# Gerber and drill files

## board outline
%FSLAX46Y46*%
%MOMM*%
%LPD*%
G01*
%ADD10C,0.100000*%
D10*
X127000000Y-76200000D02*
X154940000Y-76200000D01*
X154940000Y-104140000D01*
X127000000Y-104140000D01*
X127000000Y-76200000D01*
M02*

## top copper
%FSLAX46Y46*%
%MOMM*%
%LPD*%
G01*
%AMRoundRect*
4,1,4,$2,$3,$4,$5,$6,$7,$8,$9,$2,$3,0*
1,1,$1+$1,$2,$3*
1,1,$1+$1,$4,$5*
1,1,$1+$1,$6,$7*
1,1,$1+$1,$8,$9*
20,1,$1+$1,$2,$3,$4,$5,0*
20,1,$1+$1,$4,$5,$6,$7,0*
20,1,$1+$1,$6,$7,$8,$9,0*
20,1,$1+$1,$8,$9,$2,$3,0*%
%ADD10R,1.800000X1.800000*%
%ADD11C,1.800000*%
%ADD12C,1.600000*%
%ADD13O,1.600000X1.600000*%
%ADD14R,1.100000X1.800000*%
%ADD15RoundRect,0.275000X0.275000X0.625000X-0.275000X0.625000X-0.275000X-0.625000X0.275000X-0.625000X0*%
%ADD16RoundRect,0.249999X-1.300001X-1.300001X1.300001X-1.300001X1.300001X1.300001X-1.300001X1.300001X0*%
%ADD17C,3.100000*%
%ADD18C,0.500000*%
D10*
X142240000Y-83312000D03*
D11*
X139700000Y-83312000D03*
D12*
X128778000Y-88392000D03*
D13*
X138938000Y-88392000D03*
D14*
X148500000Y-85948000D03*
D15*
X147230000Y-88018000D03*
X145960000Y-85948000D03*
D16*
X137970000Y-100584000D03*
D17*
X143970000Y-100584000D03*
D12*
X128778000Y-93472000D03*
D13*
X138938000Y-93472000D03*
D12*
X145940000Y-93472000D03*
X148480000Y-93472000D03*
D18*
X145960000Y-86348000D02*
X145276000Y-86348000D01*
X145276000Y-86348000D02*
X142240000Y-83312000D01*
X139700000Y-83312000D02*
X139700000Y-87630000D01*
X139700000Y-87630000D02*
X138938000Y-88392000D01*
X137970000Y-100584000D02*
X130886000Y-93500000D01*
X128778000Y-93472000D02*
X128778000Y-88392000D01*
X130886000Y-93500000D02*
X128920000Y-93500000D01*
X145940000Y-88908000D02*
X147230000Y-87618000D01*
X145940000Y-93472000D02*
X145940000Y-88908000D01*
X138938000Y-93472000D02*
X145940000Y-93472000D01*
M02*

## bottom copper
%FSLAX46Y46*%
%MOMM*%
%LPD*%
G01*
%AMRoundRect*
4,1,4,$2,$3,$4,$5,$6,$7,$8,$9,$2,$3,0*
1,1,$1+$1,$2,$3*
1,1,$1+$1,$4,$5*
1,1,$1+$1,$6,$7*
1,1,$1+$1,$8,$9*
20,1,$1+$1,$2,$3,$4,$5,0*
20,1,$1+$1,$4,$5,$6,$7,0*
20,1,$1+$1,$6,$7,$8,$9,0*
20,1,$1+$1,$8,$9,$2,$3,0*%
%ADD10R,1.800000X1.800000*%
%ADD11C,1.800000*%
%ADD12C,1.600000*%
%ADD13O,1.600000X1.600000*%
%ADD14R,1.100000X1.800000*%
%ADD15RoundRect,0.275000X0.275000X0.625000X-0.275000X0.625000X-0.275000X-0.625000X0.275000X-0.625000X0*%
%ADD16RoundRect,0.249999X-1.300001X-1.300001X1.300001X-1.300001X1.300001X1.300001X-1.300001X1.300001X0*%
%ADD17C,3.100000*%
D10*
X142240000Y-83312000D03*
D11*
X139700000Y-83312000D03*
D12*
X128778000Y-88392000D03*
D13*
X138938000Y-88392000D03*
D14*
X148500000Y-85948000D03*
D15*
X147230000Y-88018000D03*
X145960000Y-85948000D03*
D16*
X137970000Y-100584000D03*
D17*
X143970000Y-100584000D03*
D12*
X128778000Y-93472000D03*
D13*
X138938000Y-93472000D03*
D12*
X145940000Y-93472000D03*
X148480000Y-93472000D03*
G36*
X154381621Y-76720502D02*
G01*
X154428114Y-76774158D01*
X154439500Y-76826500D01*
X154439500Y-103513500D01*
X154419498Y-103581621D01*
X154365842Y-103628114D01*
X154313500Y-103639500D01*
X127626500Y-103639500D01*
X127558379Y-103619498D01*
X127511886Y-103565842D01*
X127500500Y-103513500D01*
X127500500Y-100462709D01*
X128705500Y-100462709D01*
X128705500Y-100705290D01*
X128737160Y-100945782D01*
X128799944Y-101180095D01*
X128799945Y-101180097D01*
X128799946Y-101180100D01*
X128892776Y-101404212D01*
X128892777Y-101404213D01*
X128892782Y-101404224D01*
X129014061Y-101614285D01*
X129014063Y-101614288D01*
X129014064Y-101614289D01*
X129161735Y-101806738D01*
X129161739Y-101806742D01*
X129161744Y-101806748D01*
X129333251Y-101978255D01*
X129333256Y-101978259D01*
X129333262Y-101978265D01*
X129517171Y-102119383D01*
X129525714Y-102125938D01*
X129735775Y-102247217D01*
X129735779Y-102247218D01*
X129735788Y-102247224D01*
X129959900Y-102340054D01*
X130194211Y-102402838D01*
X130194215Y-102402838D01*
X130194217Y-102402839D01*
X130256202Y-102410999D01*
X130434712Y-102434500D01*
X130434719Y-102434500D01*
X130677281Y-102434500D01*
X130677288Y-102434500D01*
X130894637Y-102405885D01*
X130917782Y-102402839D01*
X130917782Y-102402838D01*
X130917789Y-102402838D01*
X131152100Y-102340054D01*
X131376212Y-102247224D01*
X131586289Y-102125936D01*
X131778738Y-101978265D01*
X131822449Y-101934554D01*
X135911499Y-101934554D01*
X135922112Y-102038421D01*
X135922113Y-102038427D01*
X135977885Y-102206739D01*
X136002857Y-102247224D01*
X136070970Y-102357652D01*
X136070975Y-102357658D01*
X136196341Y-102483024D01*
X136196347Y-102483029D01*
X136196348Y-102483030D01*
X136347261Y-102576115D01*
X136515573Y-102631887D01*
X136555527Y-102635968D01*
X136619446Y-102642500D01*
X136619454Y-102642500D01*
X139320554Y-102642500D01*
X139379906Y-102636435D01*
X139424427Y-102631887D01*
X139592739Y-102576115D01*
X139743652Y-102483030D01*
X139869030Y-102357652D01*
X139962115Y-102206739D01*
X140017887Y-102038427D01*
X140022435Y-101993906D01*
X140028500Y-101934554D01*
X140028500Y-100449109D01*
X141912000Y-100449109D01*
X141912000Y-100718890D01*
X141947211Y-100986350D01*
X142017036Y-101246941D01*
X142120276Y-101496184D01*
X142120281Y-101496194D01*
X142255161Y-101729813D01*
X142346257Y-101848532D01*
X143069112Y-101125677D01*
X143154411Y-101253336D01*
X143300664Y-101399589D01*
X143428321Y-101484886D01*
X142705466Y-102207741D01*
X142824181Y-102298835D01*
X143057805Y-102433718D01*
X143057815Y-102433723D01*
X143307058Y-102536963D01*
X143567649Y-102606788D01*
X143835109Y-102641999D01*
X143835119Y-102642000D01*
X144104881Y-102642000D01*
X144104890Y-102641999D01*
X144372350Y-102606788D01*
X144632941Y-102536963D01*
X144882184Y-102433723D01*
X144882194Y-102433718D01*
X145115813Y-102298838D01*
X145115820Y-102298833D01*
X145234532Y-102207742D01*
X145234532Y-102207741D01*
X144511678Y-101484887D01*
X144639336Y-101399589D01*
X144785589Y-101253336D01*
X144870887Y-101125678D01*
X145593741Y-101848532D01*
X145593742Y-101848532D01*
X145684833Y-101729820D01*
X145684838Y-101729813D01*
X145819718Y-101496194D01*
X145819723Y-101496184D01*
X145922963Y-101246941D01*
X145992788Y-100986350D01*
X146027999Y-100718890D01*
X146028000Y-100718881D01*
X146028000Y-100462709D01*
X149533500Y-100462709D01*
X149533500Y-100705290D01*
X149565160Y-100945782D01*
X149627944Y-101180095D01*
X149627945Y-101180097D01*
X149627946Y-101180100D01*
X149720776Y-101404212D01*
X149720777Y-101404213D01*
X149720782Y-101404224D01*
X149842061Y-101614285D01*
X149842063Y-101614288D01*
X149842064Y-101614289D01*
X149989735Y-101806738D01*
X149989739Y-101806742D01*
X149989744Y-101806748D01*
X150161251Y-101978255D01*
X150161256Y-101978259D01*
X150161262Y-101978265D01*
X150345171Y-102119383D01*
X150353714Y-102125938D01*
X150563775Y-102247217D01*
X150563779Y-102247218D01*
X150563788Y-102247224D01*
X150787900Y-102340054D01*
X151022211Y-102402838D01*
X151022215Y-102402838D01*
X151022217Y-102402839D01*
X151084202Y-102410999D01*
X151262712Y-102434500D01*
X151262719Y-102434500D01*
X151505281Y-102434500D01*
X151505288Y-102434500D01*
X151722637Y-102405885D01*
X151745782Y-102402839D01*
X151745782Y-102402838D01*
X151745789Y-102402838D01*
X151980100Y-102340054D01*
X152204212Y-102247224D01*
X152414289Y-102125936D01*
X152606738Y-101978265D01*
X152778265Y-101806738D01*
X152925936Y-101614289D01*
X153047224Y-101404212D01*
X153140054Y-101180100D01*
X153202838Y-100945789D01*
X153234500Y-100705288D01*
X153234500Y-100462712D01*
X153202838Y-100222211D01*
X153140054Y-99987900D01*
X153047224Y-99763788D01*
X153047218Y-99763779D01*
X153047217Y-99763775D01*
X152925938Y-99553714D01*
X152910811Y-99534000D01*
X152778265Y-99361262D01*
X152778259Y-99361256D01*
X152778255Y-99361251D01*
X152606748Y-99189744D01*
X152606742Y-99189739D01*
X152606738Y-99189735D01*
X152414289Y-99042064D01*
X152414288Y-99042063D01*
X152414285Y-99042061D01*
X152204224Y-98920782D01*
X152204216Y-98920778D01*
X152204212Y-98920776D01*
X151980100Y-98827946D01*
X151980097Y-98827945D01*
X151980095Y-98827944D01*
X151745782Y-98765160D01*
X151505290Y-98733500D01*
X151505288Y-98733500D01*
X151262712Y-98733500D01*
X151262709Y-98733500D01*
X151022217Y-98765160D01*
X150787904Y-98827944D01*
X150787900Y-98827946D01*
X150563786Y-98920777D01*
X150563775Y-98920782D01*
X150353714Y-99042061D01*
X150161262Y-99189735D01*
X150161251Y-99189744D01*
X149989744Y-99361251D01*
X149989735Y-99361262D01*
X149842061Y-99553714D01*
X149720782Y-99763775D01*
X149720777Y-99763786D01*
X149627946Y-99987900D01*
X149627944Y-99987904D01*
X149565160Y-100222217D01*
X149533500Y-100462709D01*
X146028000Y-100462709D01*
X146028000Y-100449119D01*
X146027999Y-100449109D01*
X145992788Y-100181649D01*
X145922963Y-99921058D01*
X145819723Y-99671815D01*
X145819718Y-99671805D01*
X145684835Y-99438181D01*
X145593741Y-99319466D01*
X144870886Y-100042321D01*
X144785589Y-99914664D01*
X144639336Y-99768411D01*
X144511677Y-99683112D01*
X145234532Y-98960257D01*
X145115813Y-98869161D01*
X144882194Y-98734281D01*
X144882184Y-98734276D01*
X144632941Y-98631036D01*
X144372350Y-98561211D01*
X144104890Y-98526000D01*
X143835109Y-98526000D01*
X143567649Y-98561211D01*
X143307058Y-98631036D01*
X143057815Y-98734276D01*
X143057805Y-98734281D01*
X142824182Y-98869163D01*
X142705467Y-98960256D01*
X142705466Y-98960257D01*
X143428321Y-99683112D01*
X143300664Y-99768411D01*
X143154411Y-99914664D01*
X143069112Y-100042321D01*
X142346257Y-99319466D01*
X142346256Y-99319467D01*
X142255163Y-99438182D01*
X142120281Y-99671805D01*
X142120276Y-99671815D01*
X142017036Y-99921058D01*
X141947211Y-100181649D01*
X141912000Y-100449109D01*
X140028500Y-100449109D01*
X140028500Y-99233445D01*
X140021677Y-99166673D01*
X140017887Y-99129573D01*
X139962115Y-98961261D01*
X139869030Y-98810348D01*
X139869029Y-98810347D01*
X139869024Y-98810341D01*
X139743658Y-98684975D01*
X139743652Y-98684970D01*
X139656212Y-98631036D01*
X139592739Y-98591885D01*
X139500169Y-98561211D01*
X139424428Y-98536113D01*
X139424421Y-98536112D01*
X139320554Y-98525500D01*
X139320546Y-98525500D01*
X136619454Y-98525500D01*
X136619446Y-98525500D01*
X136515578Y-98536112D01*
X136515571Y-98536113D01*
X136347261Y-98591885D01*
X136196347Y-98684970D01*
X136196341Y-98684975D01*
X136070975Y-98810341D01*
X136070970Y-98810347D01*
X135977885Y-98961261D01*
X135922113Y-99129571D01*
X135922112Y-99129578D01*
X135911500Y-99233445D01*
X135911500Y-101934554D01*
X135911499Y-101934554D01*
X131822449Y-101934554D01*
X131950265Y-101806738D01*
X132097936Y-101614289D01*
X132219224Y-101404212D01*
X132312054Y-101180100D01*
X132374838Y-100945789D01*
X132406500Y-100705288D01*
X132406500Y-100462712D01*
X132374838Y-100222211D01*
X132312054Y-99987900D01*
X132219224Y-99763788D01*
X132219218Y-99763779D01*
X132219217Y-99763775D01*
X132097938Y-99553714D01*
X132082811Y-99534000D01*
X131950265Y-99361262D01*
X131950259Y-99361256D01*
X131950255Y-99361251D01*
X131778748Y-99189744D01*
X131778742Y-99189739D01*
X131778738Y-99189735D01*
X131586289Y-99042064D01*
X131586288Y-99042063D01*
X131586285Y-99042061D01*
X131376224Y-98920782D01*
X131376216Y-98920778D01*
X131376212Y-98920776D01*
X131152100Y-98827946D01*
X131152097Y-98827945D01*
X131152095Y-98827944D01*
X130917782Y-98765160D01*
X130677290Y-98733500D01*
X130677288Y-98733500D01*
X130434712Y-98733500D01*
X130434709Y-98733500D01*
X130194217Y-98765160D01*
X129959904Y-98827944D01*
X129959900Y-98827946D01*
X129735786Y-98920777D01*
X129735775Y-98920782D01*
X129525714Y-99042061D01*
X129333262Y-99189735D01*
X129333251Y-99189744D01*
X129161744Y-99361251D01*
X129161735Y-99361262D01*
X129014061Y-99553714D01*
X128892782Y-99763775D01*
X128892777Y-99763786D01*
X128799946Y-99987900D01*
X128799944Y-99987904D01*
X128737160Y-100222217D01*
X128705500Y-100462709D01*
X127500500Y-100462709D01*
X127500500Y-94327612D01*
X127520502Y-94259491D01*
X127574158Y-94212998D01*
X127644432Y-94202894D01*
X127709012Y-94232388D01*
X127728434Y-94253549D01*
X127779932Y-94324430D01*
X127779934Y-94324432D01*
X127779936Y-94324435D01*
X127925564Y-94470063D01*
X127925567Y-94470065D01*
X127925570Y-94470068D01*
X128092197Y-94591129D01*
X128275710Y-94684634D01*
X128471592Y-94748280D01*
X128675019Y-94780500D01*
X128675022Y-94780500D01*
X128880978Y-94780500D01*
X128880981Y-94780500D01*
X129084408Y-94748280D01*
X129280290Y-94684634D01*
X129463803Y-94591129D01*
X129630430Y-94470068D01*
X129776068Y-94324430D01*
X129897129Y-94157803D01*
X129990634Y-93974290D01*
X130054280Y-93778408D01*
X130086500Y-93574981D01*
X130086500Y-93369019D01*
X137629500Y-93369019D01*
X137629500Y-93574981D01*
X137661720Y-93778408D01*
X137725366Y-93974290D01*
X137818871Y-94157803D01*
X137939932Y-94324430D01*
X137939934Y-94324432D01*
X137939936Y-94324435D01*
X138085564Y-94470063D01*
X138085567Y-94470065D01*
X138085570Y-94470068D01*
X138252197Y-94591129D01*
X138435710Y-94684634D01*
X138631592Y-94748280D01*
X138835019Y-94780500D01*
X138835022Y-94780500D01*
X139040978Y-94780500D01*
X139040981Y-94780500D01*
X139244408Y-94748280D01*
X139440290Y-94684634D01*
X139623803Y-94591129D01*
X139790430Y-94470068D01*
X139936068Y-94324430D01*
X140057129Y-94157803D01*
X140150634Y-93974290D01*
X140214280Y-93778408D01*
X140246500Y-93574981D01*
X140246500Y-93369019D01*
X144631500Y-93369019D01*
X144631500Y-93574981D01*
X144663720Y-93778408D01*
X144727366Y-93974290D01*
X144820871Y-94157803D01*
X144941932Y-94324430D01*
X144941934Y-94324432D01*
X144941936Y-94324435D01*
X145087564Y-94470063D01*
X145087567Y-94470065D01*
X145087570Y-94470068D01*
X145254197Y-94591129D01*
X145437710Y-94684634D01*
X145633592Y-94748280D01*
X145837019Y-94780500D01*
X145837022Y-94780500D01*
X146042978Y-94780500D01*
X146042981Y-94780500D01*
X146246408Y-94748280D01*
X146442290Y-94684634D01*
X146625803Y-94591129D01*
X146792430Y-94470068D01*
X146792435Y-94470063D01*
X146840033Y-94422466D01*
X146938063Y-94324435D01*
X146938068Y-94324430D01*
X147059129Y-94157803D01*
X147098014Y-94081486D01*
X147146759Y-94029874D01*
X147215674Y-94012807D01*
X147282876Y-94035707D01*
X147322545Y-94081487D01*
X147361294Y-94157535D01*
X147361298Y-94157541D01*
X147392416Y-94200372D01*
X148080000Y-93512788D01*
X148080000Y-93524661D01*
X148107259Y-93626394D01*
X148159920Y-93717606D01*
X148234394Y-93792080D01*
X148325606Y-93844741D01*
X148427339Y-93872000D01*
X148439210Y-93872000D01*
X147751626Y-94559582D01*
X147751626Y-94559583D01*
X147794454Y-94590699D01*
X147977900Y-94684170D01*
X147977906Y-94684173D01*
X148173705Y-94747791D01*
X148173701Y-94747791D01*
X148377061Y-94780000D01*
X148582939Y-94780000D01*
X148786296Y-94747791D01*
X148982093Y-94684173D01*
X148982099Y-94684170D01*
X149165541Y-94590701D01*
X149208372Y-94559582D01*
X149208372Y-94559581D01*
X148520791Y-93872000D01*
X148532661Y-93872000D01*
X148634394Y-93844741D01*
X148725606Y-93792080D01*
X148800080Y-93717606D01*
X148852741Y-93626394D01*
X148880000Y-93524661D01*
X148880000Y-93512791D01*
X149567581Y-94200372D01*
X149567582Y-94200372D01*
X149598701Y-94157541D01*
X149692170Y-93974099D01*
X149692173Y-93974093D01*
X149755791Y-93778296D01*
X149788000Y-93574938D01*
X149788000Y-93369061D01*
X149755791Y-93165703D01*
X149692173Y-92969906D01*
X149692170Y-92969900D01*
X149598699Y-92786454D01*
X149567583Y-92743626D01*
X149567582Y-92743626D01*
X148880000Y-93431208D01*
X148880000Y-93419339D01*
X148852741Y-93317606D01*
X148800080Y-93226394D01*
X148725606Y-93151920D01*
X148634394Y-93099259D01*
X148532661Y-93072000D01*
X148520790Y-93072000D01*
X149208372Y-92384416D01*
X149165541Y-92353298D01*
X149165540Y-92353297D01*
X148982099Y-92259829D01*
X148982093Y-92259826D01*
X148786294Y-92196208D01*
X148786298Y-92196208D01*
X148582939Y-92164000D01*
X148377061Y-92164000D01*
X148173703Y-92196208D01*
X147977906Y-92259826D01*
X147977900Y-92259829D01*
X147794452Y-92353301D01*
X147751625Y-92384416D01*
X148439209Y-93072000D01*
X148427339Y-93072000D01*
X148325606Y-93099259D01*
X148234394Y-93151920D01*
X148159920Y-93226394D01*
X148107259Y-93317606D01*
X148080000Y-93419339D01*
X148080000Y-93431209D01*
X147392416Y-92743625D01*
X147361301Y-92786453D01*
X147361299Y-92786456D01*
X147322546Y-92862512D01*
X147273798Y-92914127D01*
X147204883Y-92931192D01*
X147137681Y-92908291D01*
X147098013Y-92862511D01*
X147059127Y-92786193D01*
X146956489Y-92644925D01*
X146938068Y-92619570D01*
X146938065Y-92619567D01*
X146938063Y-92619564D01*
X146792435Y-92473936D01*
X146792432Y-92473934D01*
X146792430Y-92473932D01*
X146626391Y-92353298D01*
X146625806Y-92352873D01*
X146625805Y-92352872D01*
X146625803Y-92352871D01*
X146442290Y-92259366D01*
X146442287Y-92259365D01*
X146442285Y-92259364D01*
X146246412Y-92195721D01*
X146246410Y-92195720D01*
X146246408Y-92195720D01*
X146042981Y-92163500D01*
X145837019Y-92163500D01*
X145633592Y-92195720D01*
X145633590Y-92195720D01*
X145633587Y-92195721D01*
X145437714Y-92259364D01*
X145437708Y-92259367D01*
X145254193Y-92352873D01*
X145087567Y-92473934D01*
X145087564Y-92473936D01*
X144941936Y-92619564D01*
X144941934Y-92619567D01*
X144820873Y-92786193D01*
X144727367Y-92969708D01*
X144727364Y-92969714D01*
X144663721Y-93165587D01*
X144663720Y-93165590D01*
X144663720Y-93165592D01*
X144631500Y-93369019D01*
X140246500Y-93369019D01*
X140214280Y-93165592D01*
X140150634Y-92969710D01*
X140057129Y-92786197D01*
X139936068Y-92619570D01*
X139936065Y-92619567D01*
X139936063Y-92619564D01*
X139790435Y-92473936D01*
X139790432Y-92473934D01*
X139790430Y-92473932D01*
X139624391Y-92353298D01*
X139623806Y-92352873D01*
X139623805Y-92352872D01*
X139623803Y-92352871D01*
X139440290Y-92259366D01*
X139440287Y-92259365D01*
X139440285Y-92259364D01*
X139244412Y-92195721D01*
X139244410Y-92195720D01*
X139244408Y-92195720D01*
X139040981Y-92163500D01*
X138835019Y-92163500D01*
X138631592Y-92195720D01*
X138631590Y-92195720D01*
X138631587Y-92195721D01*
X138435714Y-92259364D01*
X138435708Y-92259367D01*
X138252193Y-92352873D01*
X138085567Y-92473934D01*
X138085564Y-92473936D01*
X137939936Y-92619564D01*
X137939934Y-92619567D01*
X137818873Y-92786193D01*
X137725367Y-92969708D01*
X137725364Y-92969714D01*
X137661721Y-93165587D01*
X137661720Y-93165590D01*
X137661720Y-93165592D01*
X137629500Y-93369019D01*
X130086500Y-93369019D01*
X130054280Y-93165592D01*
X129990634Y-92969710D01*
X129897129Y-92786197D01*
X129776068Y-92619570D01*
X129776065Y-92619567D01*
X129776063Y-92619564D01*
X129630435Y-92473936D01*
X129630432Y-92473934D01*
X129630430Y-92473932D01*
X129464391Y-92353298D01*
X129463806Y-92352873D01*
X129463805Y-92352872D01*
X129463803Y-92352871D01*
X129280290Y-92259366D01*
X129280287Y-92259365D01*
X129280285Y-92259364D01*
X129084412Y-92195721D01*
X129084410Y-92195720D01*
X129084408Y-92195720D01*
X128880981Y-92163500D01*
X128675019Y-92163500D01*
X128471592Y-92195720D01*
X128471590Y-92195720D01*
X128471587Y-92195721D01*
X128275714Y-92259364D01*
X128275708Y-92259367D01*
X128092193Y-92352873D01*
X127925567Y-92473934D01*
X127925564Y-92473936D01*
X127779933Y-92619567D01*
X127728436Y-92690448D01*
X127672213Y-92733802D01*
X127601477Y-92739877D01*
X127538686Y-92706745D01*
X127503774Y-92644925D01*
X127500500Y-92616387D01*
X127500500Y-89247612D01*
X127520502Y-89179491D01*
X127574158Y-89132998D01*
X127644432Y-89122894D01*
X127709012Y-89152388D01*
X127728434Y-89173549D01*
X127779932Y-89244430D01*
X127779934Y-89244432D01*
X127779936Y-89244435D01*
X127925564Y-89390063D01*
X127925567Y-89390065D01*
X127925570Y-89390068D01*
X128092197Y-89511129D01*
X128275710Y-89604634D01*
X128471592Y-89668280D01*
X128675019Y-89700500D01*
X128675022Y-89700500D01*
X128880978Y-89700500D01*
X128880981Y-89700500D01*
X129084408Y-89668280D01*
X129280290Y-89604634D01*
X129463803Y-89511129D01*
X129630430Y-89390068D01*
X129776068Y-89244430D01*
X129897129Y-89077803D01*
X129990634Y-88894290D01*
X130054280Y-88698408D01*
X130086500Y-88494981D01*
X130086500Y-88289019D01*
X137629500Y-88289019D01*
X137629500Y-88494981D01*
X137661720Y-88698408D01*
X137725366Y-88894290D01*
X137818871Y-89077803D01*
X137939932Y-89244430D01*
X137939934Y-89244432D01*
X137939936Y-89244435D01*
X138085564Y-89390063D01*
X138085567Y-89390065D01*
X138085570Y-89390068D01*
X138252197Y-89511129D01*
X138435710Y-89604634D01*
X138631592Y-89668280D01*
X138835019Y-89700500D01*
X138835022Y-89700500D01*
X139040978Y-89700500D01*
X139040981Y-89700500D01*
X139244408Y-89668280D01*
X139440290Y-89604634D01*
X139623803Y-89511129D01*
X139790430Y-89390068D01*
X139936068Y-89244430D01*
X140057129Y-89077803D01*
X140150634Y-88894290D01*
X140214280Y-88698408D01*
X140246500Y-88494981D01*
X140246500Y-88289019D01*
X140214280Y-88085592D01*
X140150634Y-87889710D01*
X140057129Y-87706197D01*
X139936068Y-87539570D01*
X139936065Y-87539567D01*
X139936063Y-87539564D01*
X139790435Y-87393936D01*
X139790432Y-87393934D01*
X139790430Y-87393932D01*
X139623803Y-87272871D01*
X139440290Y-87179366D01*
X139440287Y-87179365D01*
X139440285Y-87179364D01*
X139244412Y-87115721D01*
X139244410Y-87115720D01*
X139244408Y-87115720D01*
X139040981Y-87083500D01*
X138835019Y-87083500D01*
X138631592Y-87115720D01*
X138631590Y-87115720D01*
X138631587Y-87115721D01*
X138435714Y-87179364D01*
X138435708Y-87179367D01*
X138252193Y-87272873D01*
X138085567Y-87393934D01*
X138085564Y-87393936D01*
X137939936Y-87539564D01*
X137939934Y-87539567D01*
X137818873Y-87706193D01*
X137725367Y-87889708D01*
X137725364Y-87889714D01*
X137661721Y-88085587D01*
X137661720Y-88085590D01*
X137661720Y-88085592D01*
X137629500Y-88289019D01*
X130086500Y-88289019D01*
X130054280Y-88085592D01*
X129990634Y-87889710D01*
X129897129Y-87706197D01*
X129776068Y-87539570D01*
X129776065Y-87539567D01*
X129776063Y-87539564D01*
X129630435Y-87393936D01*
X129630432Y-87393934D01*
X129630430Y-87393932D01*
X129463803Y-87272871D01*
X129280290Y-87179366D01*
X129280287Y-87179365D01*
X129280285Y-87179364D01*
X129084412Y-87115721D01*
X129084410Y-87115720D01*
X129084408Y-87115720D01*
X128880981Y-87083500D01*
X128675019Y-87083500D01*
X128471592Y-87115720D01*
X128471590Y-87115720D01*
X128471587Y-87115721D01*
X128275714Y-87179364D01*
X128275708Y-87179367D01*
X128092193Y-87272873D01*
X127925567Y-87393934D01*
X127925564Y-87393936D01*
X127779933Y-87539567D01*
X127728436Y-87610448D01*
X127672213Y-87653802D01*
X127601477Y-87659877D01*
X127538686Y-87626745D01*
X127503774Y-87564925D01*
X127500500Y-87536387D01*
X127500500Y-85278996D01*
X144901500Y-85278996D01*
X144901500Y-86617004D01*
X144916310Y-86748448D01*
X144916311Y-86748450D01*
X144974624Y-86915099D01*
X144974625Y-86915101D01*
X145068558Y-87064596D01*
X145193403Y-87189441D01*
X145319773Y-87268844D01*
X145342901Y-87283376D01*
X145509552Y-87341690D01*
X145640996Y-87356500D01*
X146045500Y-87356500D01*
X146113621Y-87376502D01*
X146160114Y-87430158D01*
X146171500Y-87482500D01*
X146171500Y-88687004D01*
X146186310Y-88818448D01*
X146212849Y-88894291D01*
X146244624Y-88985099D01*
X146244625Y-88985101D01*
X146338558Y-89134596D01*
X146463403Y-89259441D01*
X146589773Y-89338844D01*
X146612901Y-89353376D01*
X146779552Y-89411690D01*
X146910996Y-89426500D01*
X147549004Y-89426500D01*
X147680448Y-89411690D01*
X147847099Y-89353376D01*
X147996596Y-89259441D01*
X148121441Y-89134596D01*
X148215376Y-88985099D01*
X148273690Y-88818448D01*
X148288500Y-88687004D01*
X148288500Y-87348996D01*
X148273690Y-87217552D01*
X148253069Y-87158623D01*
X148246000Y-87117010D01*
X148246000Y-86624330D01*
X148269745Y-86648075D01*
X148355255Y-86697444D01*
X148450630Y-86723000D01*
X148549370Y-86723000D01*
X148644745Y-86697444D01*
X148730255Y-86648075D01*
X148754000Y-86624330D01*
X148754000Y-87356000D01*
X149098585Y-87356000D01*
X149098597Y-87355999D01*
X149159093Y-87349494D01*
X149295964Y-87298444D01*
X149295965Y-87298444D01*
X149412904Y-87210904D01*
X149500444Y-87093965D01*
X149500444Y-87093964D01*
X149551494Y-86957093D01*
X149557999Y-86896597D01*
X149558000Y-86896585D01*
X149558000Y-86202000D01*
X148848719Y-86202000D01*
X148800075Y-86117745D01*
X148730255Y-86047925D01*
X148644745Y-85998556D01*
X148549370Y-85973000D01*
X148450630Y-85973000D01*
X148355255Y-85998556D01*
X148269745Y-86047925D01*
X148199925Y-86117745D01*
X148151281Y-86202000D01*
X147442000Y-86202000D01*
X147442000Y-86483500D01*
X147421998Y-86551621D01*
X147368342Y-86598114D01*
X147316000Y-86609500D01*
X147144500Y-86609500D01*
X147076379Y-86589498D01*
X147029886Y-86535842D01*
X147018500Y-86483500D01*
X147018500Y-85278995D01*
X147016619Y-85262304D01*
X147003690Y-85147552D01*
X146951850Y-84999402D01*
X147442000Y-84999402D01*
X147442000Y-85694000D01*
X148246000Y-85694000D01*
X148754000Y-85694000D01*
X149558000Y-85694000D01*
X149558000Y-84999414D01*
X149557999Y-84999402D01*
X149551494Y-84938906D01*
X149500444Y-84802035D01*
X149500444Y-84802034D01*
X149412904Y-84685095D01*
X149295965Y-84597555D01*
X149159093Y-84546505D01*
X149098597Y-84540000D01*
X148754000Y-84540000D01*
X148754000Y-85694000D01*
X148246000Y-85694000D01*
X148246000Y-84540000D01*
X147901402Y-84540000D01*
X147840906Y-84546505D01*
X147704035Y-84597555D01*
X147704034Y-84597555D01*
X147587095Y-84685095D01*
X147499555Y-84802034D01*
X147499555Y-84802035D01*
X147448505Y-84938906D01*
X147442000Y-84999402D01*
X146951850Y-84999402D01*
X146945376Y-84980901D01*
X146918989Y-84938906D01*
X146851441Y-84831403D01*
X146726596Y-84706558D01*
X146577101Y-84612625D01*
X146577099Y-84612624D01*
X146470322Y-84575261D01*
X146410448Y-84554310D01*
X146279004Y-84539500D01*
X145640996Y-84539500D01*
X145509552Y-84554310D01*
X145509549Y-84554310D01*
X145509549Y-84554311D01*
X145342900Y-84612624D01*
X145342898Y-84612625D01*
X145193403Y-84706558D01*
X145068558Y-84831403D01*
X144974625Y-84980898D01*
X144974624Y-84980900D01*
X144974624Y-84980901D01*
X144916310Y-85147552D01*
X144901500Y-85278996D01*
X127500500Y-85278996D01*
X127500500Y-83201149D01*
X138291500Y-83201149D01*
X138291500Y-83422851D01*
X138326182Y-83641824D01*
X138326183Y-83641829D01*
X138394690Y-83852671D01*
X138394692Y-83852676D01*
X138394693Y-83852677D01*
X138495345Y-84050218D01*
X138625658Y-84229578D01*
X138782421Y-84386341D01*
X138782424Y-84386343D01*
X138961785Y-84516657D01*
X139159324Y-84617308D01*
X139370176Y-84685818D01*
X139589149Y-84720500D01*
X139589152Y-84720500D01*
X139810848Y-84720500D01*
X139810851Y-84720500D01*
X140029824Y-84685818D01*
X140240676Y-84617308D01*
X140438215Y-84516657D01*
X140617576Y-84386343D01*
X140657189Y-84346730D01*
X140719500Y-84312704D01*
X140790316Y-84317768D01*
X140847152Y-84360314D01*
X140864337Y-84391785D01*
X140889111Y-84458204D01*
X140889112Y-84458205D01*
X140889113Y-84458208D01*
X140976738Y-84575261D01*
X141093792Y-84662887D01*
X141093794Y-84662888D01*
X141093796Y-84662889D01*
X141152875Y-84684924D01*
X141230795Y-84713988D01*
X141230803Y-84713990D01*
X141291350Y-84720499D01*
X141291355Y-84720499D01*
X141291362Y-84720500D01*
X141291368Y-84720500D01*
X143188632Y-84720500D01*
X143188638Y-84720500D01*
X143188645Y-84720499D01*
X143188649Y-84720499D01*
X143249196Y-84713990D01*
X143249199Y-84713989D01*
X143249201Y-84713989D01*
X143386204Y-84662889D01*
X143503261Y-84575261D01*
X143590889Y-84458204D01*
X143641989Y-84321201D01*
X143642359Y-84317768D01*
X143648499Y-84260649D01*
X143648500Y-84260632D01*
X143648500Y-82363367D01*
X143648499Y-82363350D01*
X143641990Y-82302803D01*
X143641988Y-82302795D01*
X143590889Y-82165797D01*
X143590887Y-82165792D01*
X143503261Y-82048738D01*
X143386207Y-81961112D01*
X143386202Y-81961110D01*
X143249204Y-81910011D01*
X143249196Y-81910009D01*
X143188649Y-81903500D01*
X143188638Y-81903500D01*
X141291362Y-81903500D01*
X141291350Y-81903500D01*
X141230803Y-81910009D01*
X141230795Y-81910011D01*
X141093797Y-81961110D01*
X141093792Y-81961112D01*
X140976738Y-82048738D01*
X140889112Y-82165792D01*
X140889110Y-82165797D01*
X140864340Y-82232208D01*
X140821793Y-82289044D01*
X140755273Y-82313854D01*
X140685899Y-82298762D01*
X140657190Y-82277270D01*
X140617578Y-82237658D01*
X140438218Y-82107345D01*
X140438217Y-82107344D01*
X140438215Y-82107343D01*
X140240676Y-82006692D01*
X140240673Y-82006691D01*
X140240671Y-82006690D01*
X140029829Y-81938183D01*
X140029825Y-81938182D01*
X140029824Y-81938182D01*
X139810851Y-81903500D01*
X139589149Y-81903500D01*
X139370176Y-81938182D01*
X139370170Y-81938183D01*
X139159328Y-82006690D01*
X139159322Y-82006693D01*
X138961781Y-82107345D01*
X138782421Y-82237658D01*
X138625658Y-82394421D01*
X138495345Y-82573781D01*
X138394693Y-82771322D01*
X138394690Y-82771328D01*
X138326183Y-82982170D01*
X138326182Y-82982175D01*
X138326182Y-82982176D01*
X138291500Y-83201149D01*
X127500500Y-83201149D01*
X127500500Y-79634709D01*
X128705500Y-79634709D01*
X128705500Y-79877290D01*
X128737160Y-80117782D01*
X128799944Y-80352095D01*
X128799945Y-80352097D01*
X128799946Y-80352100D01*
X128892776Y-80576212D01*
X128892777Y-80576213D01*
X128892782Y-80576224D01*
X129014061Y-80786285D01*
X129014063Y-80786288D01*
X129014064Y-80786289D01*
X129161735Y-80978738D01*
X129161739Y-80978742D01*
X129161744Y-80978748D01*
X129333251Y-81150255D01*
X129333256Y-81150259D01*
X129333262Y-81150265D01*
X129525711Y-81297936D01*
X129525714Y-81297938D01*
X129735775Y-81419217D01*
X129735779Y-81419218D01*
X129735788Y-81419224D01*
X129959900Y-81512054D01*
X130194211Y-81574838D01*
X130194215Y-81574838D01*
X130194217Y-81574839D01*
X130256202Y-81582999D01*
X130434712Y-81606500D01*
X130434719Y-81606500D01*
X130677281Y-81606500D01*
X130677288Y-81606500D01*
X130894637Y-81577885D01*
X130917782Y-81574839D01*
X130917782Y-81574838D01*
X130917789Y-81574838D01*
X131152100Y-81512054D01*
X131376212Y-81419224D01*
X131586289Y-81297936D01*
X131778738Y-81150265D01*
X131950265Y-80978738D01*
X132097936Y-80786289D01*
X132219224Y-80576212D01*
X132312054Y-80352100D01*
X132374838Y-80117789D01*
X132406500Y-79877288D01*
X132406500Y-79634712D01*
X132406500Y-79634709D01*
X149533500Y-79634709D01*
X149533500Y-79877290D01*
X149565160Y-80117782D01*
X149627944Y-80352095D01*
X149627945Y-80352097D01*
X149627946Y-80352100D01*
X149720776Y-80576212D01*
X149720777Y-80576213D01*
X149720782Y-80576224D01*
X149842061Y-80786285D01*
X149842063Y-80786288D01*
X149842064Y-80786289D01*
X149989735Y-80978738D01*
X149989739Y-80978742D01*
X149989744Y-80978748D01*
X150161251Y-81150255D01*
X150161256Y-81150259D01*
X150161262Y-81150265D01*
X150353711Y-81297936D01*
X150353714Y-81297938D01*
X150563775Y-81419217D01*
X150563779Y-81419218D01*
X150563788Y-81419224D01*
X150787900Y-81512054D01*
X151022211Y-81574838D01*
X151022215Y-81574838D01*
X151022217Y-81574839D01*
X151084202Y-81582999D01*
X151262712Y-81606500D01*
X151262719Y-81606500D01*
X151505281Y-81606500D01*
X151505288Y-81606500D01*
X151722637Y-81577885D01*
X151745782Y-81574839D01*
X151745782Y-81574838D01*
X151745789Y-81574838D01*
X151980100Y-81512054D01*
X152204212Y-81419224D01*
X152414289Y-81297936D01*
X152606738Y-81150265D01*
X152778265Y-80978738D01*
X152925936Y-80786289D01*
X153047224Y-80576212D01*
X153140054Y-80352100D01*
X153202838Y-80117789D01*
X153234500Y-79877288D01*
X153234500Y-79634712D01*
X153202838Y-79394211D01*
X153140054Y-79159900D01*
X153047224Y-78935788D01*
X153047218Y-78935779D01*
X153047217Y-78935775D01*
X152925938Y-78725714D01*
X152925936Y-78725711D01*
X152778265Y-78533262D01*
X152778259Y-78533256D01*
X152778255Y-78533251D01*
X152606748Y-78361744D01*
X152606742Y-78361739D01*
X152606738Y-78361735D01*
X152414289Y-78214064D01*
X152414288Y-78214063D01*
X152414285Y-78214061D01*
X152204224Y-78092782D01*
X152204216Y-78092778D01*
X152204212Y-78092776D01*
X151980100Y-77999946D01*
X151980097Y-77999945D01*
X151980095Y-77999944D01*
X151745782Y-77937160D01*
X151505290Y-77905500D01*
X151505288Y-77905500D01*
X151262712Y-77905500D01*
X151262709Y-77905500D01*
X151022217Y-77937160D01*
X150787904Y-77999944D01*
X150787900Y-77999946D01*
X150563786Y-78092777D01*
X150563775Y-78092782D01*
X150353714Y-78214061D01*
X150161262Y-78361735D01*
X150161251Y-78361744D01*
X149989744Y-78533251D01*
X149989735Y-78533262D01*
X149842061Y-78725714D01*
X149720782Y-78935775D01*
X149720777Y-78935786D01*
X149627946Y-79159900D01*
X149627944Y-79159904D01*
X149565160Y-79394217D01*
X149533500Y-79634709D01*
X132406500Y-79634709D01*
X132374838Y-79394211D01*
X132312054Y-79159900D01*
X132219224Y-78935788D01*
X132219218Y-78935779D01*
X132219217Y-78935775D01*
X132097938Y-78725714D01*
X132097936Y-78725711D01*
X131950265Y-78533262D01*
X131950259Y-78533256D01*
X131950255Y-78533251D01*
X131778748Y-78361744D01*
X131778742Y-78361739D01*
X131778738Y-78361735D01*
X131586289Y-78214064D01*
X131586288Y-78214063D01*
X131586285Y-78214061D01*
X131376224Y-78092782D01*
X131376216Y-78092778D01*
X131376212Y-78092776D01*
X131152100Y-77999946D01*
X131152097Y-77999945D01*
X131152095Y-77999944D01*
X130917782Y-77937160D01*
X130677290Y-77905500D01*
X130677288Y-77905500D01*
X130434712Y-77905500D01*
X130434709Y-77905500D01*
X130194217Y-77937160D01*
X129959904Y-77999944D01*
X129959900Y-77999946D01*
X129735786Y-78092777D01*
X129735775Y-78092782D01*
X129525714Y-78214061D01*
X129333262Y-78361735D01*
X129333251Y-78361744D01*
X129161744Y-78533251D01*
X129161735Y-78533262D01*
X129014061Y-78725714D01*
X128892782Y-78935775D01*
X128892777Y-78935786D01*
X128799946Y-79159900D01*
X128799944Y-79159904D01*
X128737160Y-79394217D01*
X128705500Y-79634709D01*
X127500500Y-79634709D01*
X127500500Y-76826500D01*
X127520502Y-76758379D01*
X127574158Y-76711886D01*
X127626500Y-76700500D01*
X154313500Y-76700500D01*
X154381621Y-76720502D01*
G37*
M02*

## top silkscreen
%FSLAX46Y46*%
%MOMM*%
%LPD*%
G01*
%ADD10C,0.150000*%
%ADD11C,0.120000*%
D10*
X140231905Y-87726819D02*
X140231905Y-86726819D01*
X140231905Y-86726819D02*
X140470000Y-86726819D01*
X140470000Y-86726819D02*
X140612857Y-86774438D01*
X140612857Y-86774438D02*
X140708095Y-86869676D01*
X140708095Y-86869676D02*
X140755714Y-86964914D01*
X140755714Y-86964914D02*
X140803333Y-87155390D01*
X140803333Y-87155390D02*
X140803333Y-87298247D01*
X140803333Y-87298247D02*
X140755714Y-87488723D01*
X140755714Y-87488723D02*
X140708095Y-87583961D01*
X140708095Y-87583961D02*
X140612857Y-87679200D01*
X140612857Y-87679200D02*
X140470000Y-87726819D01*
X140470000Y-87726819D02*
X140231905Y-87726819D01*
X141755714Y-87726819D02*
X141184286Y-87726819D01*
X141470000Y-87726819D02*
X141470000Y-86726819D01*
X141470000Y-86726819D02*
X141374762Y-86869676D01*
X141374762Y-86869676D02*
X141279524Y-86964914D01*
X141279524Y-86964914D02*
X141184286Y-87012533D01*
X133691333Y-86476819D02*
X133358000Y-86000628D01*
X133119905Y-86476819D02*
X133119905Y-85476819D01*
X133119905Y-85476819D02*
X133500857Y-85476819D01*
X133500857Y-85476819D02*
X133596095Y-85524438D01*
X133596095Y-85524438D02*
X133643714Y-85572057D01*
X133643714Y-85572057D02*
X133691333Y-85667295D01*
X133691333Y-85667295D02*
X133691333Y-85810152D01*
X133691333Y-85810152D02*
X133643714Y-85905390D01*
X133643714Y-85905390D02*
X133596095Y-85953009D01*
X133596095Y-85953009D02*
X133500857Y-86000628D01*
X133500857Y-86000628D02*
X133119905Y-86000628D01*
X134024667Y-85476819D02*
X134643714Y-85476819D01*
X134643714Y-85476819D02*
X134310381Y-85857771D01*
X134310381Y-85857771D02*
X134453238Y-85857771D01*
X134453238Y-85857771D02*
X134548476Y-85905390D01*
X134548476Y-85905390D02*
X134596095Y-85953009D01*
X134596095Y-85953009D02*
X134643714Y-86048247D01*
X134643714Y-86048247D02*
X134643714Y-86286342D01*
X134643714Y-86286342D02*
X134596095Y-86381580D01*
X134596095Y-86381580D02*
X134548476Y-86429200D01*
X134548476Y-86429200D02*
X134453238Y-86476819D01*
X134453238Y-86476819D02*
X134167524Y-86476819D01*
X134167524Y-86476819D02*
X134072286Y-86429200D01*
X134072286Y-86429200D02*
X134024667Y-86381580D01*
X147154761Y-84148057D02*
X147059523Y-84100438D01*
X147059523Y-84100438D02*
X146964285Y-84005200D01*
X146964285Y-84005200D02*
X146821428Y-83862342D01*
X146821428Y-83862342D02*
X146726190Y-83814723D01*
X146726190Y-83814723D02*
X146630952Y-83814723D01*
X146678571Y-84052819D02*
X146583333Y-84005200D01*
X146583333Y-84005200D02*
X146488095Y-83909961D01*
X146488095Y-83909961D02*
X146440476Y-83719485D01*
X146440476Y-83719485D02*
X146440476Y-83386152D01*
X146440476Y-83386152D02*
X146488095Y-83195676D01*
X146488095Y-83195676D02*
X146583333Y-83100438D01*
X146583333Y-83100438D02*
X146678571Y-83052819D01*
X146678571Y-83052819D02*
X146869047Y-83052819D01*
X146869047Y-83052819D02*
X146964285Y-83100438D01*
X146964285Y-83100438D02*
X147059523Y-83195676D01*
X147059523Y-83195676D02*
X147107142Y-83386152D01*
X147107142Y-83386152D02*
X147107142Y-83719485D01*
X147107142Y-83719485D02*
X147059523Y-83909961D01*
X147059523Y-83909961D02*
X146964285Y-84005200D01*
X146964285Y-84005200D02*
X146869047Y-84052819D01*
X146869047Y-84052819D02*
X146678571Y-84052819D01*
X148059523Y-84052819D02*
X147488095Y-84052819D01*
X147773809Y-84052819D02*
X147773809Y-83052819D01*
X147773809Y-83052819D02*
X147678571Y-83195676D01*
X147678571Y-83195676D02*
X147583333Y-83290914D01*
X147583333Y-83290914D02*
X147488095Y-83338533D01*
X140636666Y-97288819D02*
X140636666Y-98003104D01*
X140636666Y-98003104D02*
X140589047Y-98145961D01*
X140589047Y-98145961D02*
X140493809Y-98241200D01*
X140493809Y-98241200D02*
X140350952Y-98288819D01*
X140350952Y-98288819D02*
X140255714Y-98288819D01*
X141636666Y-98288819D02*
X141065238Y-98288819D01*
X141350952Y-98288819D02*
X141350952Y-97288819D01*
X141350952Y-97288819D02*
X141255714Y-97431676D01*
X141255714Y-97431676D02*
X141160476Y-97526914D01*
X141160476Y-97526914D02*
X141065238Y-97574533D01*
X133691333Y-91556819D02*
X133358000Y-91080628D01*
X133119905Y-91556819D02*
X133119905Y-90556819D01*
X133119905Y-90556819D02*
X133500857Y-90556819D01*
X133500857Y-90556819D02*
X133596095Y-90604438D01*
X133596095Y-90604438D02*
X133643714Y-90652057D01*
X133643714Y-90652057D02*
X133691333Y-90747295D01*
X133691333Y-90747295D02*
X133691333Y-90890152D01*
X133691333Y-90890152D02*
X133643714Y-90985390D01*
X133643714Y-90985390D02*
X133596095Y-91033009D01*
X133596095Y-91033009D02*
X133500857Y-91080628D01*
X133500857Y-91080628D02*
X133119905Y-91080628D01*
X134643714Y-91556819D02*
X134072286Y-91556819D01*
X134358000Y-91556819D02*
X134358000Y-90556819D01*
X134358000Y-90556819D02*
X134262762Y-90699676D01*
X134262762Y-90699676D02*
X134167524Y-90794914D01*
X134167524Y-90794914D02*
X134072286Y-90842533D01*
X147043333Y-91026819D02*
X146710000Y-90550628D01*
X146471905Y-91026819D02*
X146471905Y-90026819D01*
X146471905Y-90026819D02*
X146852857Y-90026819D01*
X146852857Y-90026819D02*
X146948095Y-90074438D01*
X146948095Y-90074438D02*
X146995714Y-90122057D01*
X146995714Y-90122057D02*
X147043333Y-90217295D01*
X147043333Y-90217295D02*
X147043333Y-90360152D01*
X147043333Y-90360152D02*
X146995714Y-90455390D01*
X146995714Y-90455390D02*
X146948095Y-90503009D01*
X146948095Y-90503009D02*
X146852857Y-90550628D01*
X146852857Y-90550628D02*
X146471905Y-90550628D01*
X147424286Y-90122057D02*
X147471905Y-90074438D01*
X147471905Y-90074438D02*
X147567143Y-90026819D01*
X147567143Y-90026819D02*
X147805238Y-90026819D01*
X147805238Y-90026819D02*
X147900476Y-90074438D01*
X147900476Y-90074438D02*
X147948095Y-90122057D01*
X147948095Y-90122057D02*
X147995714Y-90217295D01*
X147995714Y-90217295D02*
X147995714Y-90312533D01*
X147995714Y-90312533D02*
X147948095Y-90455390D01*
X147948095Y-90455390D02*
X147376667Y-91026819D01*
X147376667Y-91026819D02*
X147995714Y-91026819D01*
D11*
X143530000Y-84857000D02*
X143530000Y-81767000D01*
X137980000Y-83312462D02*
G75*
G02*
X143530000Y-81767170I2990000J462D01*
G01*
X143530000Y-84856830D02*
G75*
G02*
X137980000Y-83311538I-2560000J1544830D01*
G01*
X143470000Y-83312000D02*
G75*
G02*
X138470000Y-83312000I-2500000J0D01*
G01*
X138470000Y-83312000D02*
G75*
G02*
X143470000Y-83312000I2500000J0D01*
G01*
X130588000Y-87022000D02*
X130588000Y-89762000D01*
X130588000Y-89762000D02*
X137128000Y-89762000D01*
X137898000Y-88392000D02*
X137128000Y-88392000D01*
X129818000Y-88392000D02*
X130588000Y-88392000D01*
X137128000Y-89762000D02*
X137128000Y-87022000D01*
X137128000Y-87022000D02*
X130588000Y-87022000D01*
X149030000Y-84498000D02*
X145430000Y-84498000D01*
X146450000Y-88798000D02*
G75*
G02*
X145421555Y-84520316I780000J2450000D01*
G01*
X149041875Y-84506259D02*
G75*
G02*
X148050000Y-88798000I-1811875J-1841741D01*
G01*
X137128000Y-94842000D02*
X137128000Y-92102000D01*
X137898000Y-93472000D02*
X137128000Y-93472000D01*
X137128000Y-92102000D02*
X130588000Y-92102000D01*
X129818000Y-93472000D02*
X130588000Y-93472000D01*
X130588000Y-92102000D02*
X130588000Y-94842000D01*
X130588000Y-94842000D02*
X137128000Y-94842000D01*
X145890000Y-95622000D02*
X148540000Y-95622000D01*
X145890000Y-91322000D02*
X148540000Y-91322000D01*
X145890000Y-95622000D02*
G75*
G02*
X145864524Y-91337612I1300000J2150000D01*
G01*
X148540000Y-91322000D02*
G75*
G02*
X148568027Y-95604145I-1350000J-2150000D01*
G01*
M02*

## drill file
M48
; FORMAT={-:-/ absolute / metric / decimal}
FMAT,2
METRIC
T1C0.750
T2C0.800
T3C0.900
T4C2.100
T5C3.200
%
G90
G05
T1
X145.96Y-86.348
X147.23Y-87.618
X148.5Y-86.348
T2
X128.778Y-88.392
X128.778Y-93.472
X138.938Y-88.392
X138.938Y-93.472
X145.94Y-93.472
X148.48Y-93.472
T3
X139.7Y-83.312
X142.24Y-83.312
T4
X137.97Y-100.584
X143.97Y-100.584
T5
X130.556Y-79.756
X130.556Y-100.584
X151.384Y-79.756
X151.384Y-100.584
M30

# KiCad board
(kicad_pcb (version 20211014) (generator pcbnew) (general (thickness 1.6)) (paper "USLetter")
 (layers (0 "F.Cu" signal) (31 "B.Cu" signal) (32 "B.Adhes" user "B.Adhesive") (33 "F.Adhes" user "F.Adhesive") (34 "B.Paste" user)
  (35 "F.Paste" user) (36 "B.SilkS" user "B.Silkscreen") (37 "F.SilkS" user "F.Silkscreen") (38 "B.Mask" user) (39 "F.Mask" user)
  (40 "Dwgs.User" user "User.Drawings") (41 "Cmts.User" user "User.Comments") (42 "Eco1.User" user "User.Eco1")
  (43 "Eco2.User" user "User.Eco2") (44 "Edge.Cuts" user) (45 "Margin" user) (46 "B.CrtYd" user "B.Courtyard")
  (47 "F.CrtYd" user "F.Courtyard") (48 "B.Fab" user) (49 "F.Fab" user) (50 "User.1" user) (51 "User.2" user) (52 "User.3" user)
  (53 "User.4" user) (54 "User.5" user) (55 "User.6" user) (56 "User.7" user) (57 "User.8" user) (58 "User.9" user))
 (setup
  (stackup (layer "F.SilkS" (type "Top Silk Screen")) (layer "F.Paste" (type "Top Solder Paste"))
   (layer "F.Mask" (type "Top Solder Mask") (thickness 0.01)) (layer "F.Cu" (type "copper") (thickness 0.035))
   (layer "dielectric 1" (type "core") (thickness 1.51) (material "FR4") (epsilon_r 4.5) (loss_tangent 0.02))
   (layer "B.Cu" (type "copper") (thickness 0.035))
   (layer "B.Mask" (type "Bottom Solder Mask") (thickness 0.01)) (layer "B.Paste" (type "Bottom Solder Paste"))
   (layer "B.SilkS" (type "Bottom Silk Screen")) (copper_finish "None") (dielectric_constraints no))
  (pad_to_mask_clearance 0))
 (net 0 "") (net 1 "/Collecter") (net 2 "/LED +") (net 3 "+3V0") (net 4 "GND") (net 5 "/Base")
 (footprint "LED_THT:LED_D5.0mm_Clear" (layer "F.Cu") (at 142.24 83.312 180)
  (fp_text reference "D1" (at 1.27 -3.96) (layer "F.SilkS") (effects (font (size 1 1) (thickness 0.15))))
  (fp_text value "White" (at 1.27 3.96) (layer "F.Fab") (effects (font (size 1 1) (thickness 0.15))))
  (fp_line (start -1.29 -1.545) (end -1.29 1.545) (layer "F.SilkS") (width 0.12))
  (fp_arc (start 4.26 -0.000462) (mid 2.072002 2.880433) (end -1.29 1.54483) (layer "F.SilkS") (width 0.12))
  (fp_arc (start -1.29 -1.54483) (mid 2.072002 -2.880433) (end 4.26 0.000462) (layer "F.SilkS") (width 0.12))
  (fp_circle (center 1.27 0) (end 3.77 0) (layer "F.SilkS") (width 0.12) (fill none))
  (pad "1" thru_hole rect (at 0 0 180) (size 1.8 1.8) (drill 0.9) (layers *.Cu *.Mask) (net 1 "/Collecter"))
  (pad "2" thru_hole circle (at 2.54 0 180) (size 1.8 1.8) (drill 0.9) (layers *.Cu *.Mask) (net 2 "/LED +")))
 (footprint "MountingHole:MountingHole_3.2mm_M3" (layer "F.Cu") (at 130.556 100.584)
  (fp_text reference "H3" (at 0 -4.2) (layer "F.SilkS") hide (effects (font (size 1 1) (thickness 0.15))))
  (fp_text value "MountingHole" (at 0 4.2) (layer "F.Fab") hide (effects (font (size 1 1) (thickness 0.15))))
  (pad "" np_thru_hole circle (at 0 0) (size 3.2 3.2) (drill 3.2) (layers *.Cu *.Mask)))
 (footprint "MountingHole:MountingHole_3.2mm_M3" (layer "F.Cu") (at 130.556 79.756)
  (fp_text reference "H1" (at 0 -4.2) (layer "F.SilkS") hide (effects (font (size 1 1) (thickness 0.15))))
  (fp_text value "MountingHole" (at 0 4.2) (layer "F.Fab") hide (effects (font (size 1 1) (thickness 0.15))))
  (pad "" np_thru_hole circle (at 0 0) (size 3.2 3.2) (drill 3.2) (layers *.Cu *.Mask)))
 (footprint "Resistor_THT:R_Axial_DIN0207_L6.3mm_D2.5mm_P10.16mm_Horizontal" (layer "F.Cu") (at 128.778 88.392)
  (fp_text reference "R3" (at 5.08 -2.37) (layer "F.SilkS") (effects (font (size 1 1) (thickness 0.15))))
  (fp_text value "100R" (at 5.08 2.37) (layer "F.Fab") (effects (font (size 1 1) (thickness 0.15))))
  (fp_line (start 1.81 -1.37) (end 1.81 1.37) (layer "F.SilkS") (width 0.12))
  (fp_line (start 1.81 1.37) (end 8.35 1.37) (layer "F.SilkS") (width 0.12))
  (fp_line (start 9.12 0) (end 8.35 0) (layer "F.SilkS") (width 0.12))
  (fp_line (start 1.04 0) (end 1.81 0) (layer "F.SilkS") (width 0.12))
  (fp_line (start 8.35 1.37) (end 8.35 -1.37) (layer "F.SilkS") (width 0.12))
  (fp_line (start 8.35 -1.37) (end 1.81 -1.37) (layer "F.SilkS") (width 0.12))
  (pad "1" thru_hole circle (at 0 0) (size 1.6 1.6) (drill 0.8) (layers *.Cu *.Mask) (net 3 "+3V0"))
  (pad "2" thru_hole oval (at 10.16 0) (size 1.6 1.6) (drill 0.8) (layers *.Cu *.Mask) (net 2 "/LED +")))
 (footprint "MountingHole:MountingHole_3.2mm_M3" (layer "F.Cu") (at 151.384 100.584)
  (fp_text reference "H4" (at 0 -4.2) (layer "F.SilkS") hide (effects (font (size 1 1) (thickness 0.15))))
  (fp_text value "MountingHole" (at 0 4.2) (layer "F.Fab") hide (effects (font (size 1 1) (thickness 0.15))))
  (pad "" np_thru_hole circle (at 0 0) (size 3.2 3.2) (drill 3.2) (layers *.Cu *.Mask)))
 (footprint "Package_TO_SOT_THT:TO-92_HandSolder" (layer "F.Cu") (at 148.5 86.348 180)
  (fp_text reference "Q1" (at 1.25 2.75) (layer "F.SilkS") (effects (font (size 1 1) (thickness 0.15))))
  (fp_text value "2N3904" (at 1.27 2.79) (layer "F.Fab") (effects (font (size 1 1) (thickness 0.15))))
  (fp_line (start -0.53 1.85) (end 3.07 1.85) (layer "F.SilkS") (width 0.12))
  (fp_arc (start 2.05 -2.45) (mid 3.769931 -0.601036) (end 3.078445 1.827684) (layer "F.SilkS") (width 0.12))
  (fp_arc (start -0.541875 1.841741) (mid -1.247231 -0.581764) (end 0.45 -2.45) (layer "F.SilkS") (width 0.12))
  (pad "1" thru_hole rect (at 0 0 180) (size 1.1 1.8) (drill 0.75 (offset 0 0.4)) (layers *.Cu *.Mask) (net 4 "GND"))
  (pad "2" thru_hole roundrect (at 1.27 -1.27 180) (size 1.1 1.8) (drill 0.75 (offset 0 -0.4)) (layers *.Cu *.Mask) (roundrect_rratio 0.25)
   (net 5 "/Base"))
  (pad "3" thru_hole roundrect (at 2.54 0 180) (size 1.1 1.8) (drill 0.75 (offset 0 0.4)) (layers *.Cu *.Mask) (roundrect_rratio 0.25)
   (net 1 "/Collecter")))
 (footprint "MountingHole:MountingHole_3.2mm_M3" (layer "F.Cu") (at 151.384 79.756)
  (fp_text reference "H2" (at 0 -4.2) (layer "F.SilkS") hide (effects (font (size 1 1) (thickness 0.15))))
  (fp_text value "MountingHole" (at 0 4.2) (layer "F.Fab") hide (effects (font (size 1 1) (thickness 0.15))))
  (pad "" np_thru_hole circle (at 0 0) (size 3.2 3.2) (drill 3.2) (layers *.Cu *.Mask)))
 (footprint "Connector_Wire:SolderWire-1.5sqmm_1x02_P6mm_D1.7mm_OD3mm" (layer "F.Cu") (at 137.97 100.584)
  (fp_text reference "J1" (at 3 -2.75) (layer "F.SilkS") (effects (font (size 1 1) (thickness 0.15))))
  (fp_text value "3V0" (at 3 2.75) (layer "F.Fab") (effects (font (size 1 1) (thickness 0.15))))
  (pad "1" thru_hole roundrect (at 0 0) (size 3.1 3.1) (drill 2.1) (layers *.Cu *.Mask) (roundrect_rratio 0.080645) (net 3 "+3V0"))
  (pad "2" thru_hole circle (at 6 0) (size 3.1 3.1) (drill 2.1) (layers *.Cu *.Mask) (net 4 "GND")))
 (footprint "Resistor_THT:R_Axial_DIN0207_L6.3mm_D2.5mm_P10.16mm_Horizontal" (layer "F.Cu") (at 128.778 93.472)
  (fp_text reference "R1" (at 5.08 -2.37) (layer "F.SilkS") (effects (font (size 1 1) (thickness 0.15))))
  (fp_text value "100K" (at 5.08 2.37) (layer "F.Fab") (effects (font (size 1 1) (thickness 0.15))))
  (fp_line (start 8.35 1.37) (end 8.35 -1.37) (layer "F.SilkS") (width 0.12))
  (fp_line (start 9.12 0) (end 8.35 0) (layer "F.SilkS") (width 0.12))
  (fp_line (start 8.35 -1.37) (end 1.81 -1.37) (layer "F.SilkS") (width 0.12))
  (fp_line (start 1.04 0) (end 1.81 0) (layer "F.SilkS") (width 0.12))
  (fp_line (start 1.81 -1.37) (end 1.81 1.37) (layer "F.SilkS") (width 0.12))
  (fp_line (start 1.81 1.37) (end 8.35 1.37) (layer "F.SilkS") (width 0.12))
  (pad "1" thru_hole circle (at 0 0) (size 1.6 1.6) (drill 0.8) (layers *.Cu *.Mask) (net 3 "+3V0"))
  (pad "2" thru_hole oval (at 10.16 0) (size 1.6 1.6) (drill 0.8) (layers *.Cu *.Mask) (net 5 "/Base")))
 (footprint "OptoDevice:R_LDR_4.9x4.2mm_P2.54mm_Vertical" (layer "F.Cu") (at 145.94 93.472)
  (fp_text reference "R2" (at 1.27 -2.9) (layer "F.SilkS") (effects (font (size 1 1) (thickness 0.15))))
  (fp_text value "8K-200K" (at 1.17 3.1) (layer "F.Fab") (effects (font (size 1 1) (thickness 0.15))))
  (fp_line (start -0.05 2.15) (end 2.6 2.15) (layer "F.SilkS") (width 0.12))
  (fp_line (start -0.05 -2.15) (end 2.6 -2.15) (layer "F.SilkS") (width 0.12))
  (fp_arc (start -0.05 2.15) (mid -1.262424 0.01494) (end -0.075476 -2.134388) (layer "F.SilkS") (width 0.12))
  (fp_arc (start 2.6 -2.15) (mid 3.788646 -0.016616) (end 2.628027 2.132145) (layer "F.SilkS") (width 0.12))
  (pad "1" thru_hole circle (at 0 0) (size 1.6 1.6) (drill 0.8) (layers *.Cu *.Mask) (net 5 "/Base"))
  (pad "2" thru_hole circle (at 2.54 0) (size 1.6 1.6) (drill 0.8) (layers *.Cu *.Mask) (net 4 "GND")))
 (gr_rect (start 127 76.2) (end 154.94 104.14) (layer "Edge.Cuts") (width 0.1) (fill none))
 (segment (start 145.96 86.348) (end 145.276 86.348) (width 0.5) (layer "F.Cu") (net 1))
 (segment (start 145.276 86.348) (end 142.24 83.312) (width 0.5) (layer "F.Cu") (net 1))
 (segment (start 139.7 83.312) (end 139.7 87.63) (width 0.5) (layer "F.Cu") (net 2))
 (segment (start 139.7 87.63) (end 138.938 88.392) (width 0.5) (layer "F.Cu") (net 2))
 (segment (start 137.97 100.584) (end 130.886 93.5) (width 0.5) (layer "F.Cu") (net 3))
 (segment (start 128.778 93.472) (end 128.778 88.392) (width 0.5) (layer "F.Cu") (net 3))
 (segment (start 130.886 93.5) (end 128.92 93.5) (width 0.5) (layer "F.Cu") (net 3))
 (segment (start 145.94 88.908) (end 147.23 87.618) (width 0.5) (layer "F.Cu") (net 5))
 (segment (start 145.94 93.472) (end 145.94 88.908) (width 0.5) (layer "F.Cu") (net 5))
 (segment (start 138.938 93.472) (end 145.94 93.472) (width 0.5) (layer "F.Cu") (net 5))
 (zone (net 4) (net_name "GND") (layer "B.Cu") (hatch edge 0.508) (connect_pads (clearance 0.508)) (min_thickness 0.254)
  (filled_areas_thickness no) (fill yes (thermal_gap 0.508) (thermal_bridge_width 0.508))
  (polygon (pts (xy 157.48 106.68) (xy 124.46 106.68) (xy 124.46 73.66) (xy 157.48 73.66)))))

